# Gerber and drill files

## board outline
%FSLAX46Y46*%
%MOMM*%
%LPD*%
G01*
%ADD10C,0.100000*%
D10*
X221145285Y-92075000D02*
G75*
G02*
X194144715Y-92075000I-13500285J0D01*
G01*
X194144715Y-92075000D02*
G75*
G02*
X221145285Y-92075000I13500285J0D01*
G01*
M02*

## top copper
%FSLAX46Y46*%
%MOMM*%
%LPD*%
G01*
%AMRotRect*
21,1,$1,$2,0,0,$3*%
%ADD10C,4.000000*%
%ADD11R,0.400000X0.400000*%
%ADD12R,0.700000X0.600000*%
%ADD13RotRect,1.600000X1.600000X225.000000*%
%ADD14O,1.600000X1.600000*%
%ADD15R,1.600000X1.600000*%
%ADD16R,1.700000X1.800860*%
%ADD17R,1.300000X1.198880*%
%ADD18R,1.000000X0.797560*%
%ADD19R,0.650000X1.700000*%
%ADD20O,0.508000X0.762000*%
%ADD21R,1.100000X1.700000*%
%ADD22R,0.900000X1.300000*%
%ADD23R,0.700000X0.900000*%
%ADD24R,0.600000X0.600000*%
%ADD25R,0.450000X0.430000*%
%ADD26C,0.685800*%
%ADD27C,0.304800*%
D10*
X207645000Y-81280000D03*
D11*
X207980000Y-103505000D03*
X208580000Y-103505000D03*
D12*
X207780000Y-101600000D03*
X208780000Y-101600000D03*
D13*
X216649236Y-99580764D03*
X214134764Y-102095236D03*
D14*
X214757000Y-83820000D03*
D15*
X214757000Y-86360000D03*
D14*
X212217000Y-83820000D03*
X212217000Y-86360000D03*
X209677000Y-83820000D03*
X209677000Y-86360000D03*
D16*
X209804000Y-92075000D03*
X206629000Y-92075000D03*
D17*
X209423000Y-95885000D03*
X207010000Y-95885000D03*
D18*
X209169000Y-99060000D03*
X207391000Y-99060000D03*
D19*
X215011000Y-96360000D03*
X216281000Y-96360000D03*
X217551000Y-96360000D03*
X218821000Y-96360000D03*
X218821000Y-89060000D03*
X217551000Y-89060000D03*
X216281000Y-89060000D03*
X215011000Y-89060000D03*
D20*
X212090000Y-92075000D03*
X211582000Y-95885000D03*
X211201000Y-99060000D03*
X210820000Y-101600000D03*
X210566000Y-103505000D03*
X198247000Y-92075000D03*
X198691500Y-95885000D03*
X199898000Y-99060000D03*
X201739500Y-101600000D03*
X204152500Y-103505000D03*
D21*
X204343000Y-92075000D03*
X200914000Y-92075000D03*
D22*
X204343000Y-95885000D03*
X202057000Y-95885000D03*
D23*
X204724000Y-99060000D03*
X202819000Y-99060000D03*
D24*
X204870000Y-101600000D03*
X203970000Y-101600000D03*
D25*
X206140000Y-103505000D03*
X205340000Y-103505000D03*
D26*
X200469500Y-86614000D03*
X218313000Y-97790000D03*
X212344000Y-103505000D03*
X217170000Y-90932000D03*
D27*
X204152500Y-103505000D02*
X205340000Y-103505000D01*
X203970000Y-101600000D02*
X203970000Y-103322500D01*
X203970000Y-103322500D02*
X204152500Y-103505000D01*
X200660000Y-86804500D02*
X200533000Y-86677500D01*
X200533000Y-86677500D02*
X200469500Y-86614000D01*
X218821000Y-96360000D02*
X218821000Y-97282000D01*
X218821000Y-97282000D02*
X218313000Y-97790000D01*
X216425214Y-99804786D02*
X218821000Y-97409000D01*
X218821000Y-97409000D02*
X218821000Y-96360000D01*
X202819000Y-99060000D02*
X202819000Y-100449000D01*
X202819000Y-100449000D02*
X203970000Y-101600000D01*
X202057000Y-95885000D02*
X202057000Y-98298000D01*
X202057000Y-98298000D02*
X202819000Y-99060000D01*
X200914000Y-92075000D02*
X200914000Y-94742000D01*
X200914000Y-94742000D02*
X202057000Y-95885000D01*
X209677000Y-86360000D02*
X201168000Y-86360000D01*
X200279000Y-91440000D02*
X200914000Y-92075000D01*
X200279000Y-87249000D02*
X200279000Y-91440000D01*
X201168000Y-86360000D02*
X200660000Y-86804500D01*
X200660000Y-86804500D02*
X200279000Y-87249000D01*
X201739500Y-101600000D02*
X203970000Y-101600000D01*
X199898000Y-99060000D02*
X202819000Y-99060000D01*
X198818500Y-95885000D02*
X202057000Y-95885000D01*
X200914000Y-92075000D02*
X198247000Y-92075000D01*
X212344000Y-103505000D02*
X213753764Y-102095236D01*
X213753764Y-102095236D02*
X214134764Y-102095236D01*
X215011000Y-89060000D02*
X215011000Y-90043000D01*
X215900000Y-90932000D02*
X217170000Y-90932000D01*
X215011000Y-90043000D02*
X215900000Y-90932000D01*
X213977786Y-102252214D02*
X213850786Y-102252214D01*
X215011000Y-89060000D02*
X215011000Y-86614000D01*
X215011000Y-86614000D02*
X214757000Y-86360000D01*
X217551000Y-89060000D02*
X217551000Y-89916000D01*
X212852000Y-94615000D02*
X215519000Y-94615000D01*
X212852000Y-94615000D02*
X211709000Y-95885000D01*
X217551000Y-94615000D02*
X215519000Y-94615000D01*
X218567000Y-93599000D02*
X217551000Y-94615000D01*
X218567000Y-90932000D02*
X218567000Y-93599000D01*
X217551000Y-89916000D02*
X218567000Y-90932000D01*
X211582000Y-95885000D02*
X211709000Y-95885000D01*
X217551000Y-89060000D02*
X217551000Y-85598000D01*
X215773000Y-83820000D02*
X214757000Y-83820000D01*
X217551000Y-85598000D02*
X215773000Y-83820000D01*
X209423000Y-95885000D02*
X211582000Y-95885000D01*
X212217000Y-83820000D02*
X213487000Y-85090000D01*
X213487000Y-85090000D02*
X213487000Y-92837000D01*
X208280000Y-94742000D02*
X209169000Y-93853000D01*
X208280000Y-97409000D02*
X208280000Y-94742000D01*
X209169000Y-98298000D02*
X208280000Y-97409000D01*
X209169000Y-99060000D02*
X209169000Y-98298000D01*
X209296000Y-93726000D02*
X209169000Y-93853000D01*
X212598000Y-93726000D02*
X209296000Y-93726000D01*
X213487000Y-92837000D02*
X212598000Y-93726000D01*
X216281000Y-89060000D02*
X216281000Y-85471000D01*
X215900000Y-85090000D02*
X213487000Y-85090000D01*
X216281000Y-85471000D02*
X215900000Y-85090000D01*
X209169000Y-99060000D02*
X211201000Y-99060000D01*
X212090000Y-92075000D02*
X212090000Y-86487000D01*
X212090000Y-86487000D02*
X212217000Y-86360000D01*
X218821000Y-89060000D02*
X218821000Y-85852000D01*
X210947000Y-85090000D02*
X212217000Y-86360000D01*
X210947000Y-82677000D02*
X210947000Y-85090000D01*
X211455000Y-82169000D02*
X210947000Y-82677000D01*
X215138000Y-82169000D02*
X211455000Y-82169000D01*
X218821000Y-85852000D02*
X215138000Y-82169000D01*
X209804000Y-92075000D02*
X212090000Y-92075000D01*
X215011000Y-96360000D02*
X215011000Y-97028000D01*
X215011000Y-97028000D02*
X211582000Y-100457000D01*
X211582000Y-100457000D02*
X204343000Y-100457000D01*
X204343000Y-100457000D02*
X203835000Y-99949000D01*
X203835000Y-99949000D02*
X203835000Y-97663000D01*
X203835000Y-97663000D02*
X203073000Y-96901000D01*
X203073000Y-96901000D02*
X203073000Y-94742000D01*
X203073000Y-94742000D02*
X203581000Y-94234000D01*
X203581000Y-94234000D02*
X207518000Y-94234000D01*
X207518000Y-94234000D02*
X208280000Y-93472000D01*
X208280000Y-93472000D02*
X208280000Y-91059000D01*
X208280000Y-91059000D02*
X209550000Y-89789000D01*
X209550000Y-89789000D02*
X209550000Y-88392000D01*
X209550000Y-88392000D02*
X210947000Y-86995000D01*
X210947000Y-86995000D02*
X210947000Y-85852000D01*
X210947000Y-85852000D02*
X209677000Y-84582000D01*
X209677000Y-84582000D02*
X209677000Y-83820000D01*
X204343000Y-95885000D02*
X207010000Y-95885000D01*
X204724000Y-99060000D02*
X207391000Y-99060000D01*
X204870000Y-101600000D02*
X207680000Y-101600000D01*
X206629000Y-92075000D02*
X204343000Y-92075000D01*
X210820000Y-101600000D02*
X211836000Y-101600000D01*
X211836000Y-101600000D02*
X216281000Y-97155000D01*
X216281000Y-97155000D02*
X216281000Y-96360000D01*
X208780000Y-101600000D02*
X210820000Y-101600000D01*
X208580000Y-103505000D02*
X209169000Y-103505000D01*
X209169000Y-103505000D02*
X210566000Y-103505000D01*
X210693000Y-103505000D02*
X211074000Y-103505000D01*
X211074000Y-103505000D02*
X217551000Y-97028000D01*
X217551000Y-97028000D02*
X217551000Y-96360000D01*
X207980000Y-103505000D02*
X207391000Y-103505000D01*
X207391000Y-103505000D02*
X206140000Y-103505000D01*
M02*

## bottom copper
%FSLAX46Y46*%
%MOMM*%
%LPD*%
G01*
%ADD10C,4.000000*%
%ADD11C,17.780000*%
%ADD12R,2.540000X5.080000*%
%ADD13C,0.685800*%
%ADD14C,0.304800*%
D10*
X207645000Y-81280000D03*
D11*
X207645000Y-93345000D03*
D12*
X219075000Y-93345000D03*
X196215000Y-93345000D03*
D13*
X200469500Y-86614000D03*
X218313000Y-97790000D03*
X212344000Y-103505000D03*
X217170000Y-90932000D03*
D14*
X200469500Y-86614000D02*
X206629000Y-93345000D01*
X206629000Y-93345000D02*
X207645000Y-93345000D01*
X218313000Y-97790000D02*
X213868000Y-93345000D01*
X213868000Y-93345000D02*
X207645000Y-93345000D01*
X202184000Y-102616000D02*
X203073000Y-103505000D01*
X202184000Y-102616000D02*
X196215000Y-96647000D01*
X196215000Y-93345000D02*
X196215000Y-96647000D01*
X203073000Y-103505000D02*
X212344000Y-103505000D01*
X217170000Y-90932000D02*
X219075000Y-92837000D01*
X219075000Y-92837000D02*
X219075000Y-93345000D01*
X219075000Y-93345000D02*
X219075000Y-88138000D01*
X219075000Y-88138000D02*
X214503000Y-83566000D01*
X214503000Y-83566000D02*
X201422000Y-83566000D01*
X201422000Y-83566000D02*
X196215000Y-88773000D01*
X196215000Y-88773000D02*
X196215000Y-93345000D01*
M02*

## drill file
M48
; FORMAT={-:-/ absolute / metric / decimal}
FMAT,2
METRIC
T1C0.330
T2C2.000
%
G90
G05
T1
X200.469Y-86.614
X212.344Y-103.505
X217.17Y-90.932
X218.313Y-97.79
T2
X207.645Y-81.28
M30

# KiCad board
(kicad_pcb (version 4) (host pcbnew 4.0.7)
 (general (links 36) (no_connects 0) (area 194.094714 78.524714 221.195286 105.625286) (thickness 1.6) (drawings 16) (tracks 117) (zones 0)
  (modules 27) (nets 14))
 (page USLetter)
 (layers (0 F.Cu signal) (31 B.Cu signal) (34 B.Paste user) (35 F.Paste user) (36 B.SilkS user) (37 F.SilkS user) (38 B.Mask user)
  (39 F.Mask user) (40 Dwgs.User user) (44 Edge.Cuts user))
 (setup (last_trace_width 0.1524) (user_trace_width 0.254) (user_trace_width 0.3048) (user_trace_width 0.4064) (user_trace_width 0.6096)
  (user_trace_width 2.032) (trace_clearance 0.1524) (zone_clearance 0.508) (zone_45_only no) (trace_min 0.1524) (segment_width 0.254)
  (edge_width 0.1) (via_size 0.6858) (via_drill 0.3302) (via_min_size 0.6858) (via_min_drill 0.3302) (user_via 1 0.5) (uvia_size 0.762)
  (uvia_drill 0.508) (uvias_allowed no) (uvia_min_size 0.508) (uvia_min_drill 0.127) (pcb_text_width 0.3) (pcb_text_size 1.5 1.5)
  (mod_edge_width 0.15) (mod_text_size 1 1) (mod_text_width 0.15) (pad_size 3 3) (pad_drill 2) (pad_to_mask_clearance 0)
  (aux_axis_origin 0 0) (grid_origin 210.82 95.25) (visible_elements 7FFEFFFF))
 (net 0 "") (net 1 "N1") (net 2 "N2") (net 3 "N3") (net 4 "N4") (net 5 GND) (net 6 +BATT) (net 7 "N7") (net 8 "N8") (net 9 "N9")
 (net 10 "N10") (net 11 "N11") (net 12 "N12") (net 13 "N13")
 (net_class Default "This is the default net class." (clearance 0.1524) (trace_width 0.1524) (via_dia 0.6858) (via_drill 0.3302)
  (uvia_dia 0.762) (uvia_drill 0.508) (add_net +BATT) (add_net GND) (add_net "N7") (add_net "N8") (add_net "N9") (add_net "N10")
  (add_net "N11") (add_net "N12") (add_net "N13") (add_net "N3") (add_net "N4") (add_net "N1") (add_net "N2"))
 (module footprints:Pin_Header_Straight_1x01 (layer F.Cu) (at 207.645 81.28)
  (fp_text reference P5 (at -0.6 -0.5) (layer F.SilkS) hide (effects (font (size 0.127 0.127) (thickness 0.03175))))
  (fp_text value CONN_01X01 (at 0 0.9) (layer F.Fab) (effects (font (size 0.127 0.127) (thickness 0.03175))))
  (pad 1 thru_hole circle (at 0 0) (size 4 4) (drill 2) (layers *.Cu *.Mask)))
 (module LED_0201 (layer F.Cu) (at 208.28 103.505)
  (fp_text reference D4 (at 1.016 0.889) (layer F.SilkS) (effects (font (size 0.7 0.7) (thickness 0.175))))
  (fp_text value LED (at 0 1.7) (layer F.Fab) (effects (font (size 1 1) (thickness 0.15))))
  (pad 1 smd rect (at -0.3 0) (size 0.4 0.4) (layers F.Cu F.Paste F.Mask) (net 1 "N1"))
  (pad 2 smd rect (at 0.3 0) (size 0.4 0.4) (layers F.Cu F.Paste F.Mask) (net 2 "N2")))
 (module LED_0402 (layer F.Cu) (at 208.28 101.6)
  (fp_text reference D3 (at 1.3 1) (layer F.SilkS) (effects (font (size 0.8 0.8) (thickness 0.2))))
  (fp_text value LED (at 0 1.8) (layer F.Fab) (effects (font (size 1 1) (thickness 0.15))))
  (pad 1 smd rect (at -0.5 0) (size 0.7 0.6) (layers F.Cu F.Paste F.Mask) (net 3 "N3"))
  (pad 2 smd rect (at 0.5 0) (size 0.7 0.6) (layers F.Cu F.Paste F.Mask) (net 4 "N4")))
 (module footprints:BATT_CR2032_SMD (layer B.Cu) (at 207.645 93.345 180)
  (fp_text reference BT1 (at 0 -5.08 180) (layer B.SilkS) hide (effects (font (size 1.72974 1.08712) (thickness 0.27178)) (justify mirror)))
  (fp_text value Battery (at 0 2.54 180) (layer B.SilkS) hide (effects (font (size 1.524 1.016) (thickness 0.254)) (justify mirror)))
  (pad 2 smd circle (at 0 0 180) (size 17.78 17.78) (layers B.Cu B.Paste B.Mask) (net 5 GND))
  (pad 1 smd rect (at -11.43 0 180) (size 2.54 5.08) (layers B.Cu B.Paste B.Mask) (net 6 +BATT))
  (pad 1 smd rect (at 11.43 0 180) (size 2.54 5.08) (layers B.Cu B.Paste B.Mask) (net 6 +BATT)))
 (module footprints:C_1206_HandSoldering (layer F.Cu) (at 215.392 100.838 225)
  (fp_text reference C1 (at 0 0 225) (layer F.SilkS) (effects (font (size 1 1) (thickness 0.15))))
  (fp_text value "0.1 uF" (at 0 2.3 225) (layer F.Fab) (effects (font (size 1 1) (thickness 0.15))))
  (pad 1 smd rect (at -1.778 0 225) (size 1.6 1.6) (layers F.Cu F.Paste F.Mask) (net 5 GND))
  (pad 2 smd rect (at 1.778 0 225) (size 1.6 1.6) (layers F.Cu F.Paste F.Mask) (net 6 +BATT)))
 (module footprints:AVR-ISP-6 (layer F.Cu) (at 214.757 83.82 270)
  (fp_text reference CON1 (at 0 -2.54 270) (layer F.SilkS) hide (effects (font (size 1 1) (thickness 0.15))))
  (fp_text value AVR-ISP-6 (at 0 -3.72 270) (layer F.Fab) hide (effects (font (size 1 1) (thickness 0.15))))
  (pad 1 smd oval (at 0 0 270) (size 1.6 1.6) (layers F.Cu F.Paste F.Mask) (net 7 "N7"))
  (pad 2 smd rect (at 2.54 0 270) (size 1.6 1.6) (layers F.Cu F.Paste F.Mask) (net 6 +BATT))
  (pad 3 smd oval (at 0 2.54 270) (size 1.6 1.6) (layers F.Cu F.Paste F.Mask) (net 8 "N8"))
  (pad 4 smd oval (at 2.54 2.54 270) (size 1.6 1.6) (layers F.Cu F.Paste F.Mask) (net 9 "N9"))
  (pad 5 smd oval (at 0 5.08 270) (size 1.6 1.6) (layers F.Cu F.Paste F.Mask) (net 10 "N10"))
  (pad 6 smd oval (at 2.54 5.08 270) (size 1.6 1.6) (layers F.Cu F.Paste F.Mask) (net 5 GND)))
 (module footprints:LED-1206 (layer F.Cu) (at 208.28 92.075)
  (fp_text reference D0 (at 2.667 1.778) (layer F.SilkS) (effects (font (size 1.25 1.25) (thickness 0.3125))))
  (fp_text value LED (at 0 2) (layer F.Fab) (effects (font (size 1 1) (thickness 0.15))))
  (pad 2 smd rect (at 1.524 0 180) (size 1.7 1.80086) (layers F.Cu F.Paste F.Mask) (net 9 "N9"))
  (pad 1 smd rect (at -1.651 0 180) (size 1.7 1.80086) (layers F.Cu F.Paste F.Mask) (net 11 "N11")))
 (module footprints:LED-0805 (layer F.Cu) (at 208.28 95.885)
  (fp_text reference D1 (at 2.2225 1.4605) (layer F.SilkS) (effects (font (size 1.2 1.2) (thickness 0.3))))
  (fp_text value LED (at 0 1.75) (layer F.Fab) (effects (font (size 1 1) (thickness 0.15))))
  (pad 2 smd rect (at 1.143 0 180) (size 1.3 1.19888) (layers F.Cu F.Paste F.Mask) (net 7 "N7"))
  (pad 1 smd rect (at -1.27 0 180) (size 1.3 1.19888) (layers F.Cu F.Paste F.Mask) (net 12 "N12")))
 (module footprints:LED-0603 (layer F.Cu) (at 208.28 99.06)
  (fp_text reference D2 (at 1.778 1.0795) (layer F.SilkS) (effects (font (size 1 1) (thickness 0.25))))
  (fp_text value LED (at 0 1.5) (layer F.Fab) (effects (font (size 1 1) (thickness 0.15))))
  (pad 2 smd rect (at 0.889 0 180) (size 1 0.79756) (layers F.Cu F.Paste F.Mask) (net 8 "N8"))
  (pad 1 smd rect (at -0.889 0 180) (size 1 0.79756) (layers F.Cu F.Paste F.Mask) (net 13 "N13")))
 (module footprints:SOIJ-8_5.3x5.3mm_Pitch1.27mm (layer F.Cu) (at 216.916 92.71 90)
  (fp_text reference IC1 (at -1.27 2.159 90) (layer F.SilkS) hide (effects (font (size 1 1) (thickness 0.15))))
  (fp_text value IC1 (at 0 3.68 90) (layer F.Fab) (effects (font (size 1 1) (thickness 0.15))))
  (pad 1 smd rect (at -3.65 -1.905 90) (size 1.7 0.65) (layers F.Cu F.Paste F.Mask) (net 10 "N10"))
  (pad 2 smd rect (at -3.65 -0.635 90) (size 1.7 0.65) (layers F.Cu F.Paste F.Mask) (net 4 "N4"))
  (pad 3 smd rect (at -3.65 0.635 90) (size 1.7 0.65) (layers F.Cu F.Paste F.Mask) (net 2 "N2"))
  (pad 4 smd rect (at -3.65 1.905 90) (size 1.7 0.65) (layers F.Cu F.Paste F.Mask) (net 5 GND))
  (pad 5 smd rect (at 3.65 1.905 90) (size 1.7 0.65) (layers F.Cu F.Paste F.Mask) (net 9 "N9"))
  (pad 6 smd rect (at 3.65 0.635 90) (size 1.7 0.65) (layers F.Cu F.Paste F.Mask) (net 7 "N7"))
  (pad 7 smd rect (at 3.65 -0.635 90) (size 1.7 0.65) (layers F.Cu F.Paste F.Mask) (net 8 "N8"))
  (pad 8 smd rect (at 3.65 -1.905 90) (size 1.7 0.65) (layers F.Cu F.Paste F.Mask) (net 6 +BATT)))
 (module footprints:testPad (layer F.Cu) (at 212.09 92.075)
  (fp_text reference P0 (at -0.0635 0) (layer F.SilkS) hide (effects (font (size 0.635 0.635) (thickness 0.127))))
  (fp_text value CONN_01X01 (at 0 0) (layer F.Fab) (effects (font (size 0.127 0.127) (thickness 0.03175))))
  (pad 1 smd oval (at 0 0) (size 0.508 0.762) (layers F.Cu F.Paste F.Mask) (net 9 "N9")))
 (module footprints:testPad (layer F.Cu) (at 211.582 95.885)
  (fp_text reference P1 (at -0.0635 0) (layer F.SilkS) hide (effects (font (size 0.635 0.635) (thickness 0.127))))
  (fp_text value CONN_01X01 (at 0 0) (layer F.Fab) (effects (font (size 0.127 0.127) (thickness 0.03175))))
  (pad 1 smd oval (at 0 0) (size 0.508 0.762) (layers F.Cu F.Paste F.Mask) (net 7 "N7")))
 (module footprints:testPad (layer F.Cu) (at 211.201 99.06)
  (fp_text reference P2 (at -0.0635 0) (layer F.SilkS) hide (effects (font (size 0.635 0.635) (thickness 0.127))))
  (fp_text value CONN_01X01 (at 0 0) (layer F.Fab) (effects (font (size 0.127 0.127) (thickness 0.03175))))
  (pad 1 smd oval (at 0 0) (size 0.508 0.762) (layers F.Cu F.Paste F.Mask) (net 8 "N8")))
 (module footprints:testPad (layer F.Cu) (at 210.82 101.6)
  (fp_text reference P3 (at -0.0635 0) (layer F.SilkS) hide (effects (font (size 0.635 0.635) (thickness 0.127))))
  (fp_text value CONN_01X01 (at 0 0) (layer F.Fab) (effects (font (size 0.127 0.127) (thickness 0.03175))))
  (pad 1 smd oval (at 0 0) (size 0.508 0.762) (layers F.Cu F.Paste F.Mask) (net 4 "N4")))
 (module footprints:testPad (layer F.Cu) (at 210.566 103.505)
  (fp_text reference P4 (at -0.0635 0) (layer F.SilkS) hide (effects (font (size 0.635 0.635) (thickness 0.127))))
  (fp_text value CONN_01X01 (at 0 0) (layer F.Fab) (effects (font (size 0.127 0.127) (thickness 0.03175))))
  (pad 1 smd oval (at 0 0) (size 0.508 0.762) (layers F.Cu F.Paste F.Mask) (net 2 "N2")))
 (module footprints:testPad (layer F.Cu) (at 198.247 92.075)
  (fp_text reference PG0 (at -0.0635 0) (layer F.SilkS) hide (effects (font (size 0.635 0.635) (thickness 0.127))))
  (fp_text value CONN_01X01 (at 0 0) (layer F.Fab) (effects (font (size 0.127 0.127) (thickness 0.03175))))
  (pad 1 smd oval (at 0 0) (size 0.508 0.762) (layers F.Cu F.Paste F.Mask) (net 5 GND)))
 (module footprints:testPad (layer F.Cu) (at 198.6915 95.885)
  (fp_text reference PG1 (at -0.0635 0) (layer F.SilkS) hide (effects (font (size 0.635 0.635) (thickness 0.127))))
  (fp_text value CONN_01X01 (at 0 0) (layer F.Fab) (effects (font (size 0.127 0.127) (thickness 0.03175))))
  (pad 1 smd oval (at 0 0) (size 0.508 0.762) (layers F.Cu F.Paste F.Mask) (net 5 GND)))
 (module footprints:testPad (layer F.Cu) (at 199.898 99.06)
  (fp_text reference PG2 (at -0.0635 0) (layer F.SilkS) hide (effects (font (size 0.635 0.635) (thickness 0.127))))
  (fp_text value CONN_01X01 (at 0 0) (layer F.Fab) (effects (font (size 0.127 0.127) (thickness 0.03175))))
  (pad 1 smd oval (at 0 0) (size 0.508 0.762) (layers F.Cu F.Paste F.Mask) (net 5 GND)))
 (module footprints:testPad (layer F.Cu) (at 201.7395 101.6)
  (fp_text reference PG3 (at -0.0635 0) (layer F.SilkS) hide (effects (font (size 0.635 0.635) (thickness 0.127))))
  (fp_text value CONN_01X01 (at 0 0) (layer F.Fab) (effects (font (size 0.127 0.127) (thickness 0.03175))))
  (pad 1 smd oval (at 0 0) (size 0.508 0.762) (layers F.Cu F.Paste F.Mask) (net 5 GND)))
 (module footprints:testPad (layer F.Cu) (at 204.1525 103.505)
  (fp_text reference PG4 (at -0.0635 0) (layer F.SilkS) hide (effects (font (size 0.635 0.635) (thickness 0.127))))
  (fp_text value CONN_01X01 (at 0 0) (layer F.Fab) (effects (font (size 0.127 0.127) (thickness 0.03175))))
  (pad 1 smd oval (at 0 0) (size 0.508 0.762) (layers F.Cu F.Paste F.Mask) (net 5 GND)))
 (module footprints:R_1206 (layer F.Cu) (at 202.565 92.075 180)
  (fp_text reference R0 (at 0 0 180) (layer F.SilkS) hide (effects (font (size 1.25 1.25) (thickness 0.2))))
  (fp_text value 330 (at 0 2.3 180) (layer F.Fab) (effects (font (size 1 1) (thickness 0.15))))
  (pad 1 smd rect (at -1.778 0 180) (size 1.1 1.7) (layers F.Cu F.Paste F.Mask) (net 11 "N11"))
  (pad 2 smd rect (at 1.651 0 180) (size 1.1 1.7) (layers F.Cu F.Paste F.Mask) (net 5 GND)))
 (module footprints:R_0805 (layer F.Cu) (at 203.2 95.885 180)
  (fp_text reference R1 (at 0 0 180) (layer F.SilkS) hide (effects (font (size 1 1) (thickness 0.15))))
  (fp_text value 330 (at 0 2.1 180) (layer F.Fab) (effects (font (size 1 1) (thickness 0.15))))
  (pad 1 smd rect (at -1.143 0 180) (size 0.9 1.3) (layers F.Cu F.Paste F.Mask) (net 12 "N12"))
  (pad 2 smd rect (at 1.143 0 180) (size 0.9 1.3) (layers F.Cu F.Paste F.Mask) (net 5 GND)))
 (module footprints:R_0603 (layer F.Cu) (at 203.835 99.06 180)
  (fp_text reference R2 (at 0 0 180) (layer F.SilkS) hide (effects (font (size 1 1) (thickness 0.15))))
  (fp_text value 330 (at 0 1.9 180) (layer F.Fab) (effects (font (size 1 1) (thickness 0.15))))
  (pad 1 smd rect (at -0.889 0 180) (size 0.7 0.9) (layers F.Cu F.Paste F.Mask) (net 13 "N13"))
  (pad 2 smd rect (at 1.016 0 180) (size 0.7 0.9) (layers F.Cu F.Paste F.Mask) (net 5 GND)))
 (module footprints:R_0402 (layer F.Cu) (at 204.47 101.6 180)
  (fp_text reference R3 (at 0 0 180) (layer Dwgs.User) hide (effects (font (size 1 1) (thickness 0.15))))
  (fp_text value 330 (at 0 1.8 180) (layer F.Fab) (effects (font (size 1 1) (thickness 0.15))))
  (pad 1 smd rect (at -0.4 0 180) (size 0.6 0.6) (layers F.Cu F.Paste F.Mask) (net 3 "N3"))
  (pad 2 smd rect (at 0.5 0 180) (size 0.6 0.6) (layers F.Cu F.Paste F.Mask) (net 5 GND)))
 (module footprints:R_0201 (layer F.Cu) (at 205.74 103.505 180)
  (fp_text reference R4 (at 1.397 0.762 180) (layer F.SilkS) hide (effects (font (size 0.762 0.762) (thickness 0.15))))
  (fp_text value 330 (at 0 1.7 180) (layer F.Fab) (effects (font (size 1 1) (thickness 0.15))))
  (pad 1 smd rect (at -0.4 0 180) (size 0.45 0.43) (layers F.Cu F.Paste F.Mask) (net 1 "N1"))
  (pad 2 smd rect (at 0.4 0 180) (size 0.45 0.43) (layers F.Cu F.Paste F.Mask) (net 5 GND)))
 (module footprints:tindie (layer F.Cu) (at 208.534 88.9)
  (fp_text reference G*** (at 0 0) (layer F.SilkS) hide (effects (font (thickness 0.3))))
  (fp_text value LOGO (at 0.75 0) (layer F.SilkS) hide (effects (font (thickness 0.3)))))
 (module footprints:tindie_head (layer F.Cu) (at 200.914 86.36)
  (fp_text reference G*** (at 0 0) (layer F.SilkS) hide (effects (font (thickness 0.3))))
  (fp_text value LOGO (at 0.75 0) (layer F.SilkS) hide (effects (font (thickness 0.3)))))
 (gr_circle (center 207.645 92.075) (end 197.485 83.185) (layer Edge.Cuts) (width 0.1))
 (segment (start 204.1525 103.505) (end 205.34 103.505) (width 0.3048) (layer F.Cu) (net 5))
 (segment (start 203.97 101.6) (end 203.97 103.3225) (width 0.3048) (layer F.Cu) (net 5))
 (segment (start 203.97 103.3225) (end 204.1525 103.505) (width 0.3048) (layer F.Cu) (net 5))
 (segment (start 200.66 86.8045) (end 200.533 86.6775) (width 0.3048) (layer F.Cu) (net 5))
 (segment (start 200.4695 86.614) (end 206.629 93.345) (width 0.3048) (layer B.Cu) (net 5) (status 20))
 (via (at 200.4695 86.614) (size 0.6858) (drill 0.3302) (layers F.Cu B.Cu) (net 5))
 (segment (start 200.533 86.6775) (end 200.4695 86.614) (width 0.3048) (layer F.Cu) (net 5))
 (segment (start 206.629 93.345) (end 207.645 93.345) (width 0.3048) (layer B.Cu) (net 5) (status 30))
 (segment (start 218.821 96.36) (end 218.821 97.282) (width 0.3048) (layer F.Cu) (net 5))
 (segment (start 218.313 97.79) (end 213.868 93.345) (width 0.3048) (layer B.Cu) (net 5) (status 20))
 (via (at 218.313 97.79) (size 0.6858) (drill 0.3302) (layers F.Cu B.Cu) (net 5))
 (segment (start 218.821 97.282) (end 218.313 97.79) (width 0.3048) (layer F.Cu) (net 5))
 (segment (start 213.868 93.345) (end 207.645 93.345) (width 0.3048) (layer B.Cu) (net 5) (status 30))
 (segment (start 216.425214 99.804786) (end 218.821 97.409) (width 0.3048) (layer F.Cu) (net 5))
 (segment (start 218.821 97.409) (end 218.821 96.36) (width 0.3048) (layer F.Cu) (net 5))
 (segment (start 202.819 99.06) (end 202.819 100.449) (width 0.3048) (layer F.Cu) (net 5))
 (segment (start 202.819 100.449) (end 203.97 101.6) (width 0.3048) (layer F.Cu) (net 5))
 (segment (start 202.057 95.885) (end 202.057 98.298) (width 0.3048) (layer F.Cu) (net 5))
 (segment (start 202.057 98.298) (end 202.819 99.06) (width 0.3048) (layer F.Cu) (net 5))
 (segment (start 200.914 92.075) (end 200.914 94.742) (width 0.3048) (layer F.Cu) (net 5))
 (segment (start 200.914 94.742) (end 202.057 95.885) (width 0.3048) (layer F.Cu) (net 5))
 (segment (start 209.677 86.36) (end 201.168 86.36) (width 0.3048) (layer F.Cu) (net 5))
 (segment (start 200.279 91.44) (end 200.914 92.075) (width 0.3048) (layer F.Cu) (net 5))
 (segment (start 200.279 87.249) (end 200.279 91.44) (width 0.3048) (layer F.Cu) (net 5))
 (segment (start 201.168 86.36) (end 200.66 86.8045) (width 0.3048) (layer F.Cu) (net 5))
 (segment (start 200.66 86.8045) (end 200.279 87.249) (width 0.3048) (layer F.Cu) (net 5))
 (segment (start 201.7395 101.6) (end 203.97 101.6) (width 0.3048) (layer F.Cu) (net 5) (status 10))
 (segment (start 199.898 99.06) (end 202.819 99.06) (width 0.3048) (layer F.Cu) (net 5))
 (segment (start 198.8185 95.885) (end 202.057 95.885) (width 0.3048) (layer F.Cu) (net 5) (status 10))
 (segment (start 200.914 92.075) (end 198.247 92.075) (width 0.3048) (layer F.Cu) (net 5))
 (segment (start 202.184 102.616) (end 203.073 103.505) (width 0.3048) (layer B.Cu) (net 6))
 (segment (start 202.184 102.616) (end 196.215 96.647) (width 0.3048) (layer B.Cu) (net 6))
 (segment (start 196.215 93.345) (end 196.215 96.647) (width 0.3048) (layer B.Cu) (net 6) (status 10))
 (segment (start 212.344 103.505) (end 213.753764 102.095236) (width 0.3048) (layer F.Cu) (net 6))
 (via (at 212.344 103.505) (size 0.6858) (drill 0.3302) (layers F.Cu B.Cu) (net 6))
 (segment (start 203.073 103.505) (end 212.344 103.505) (width 0.3048) (layer B.Cu) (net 6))
 (segment (start 213.753764 102.095236) (end 214.134764 102.095236) (width 0.3048) (layer F.Cu) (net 6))
 (segment (start 215.011 89.06) (end 215.011 90.043) (width 0.3048) (layer F.Cu) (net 6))
 (segment (start 217.17 90.932) (end 219.075 92.837) (width 0.3048) (layer B.Cu) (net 6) (status 20))
 (via (at 217.17 90.932) (size 0.6858) (drill 0.3302) (layers F.Cu B.Cu) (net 6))
 (segment (start 215.9 90.932) (end 217.17 90.932) (width 0.3048) (layer F.Cu) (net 6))
 (segment (start 215.011 90.043) (end 215.9 90.932) (width 0.3048) (layer F.Cu) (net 6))
 (segment (start 219.075 92.837) (end 219.075 93.345) (width 0.3048) (layer B.Cu) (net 6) (status 30))
 (segment (start 219.075 93.345) (end 219.075 88.138) (width 0.3048) (layer B.Cu) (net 6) (status 10))
 (segment (start 219.075 88.138) (end 214.503 83.566) (width 0.3048) (layer B.Cu) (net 6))
 (segment (start 214.503 83.566) (end 201.422 83.566) (width 0.3048) (layer B.Cu) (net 6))
 (segment (start 201.422 83.566) (end 196.215 88.773) (width 0.3048) (layer B.Cu) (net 6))
 (segment (start 196.215 88.773) (end 196.215 93.345) (width 0.3048) (layer B.Cu) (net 6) (status 20))
 (segment (start 213.977786 102.252214) (end 213.850786 102.252214) (width 0.3048) (layer F.Cu) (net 6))
 (segment (start 215.011 89.06) (end 215.011 86.614) (width 0.3048) (layer F.Cu) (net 6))
 (segment (start 215.011 86.614) (end 214.757 86.36) (width 0.3048) (layer F.Cu) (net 6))
 (segment (start 217.551 89.06) (end 217.551 89.916) (width 0.3048) (layer F.Cu) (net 7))
 (segment (start 212.852 94.615) (end 215.519 94.615) (width 0.3048) (layer F.Cu) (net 7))
 (segment (start 212.852 94.615) (end 211.709 95.885) (width 0.3048) (layer F.Cu) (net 7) (status 20))
 (segment (start 217.551 94.615) (end 215.519 94.615) (width 0.3048) (layer F.Cu) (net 7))
 (segment (start 218.567 93.599) (end 217.551 94.615) (width 0.3048) (layer F.Cu) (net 7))
 (segment (start 218.567 90.932) (end 218.567 93.599) (width 0.3048) (layer F.Cu) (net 7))
 (segment (start 217.551 89.916) (end 218.567 90.932) (width 0.3048) (layer F.Cu) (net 7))
 (segment (start 211.582 95.885) (end 211.709 95.885) (width 0.3048) (layer F.Cu) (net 7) (status 30))
 (segment (start 217.551 89.06) (end 217.551 85.598) (width 0.3048) (layer F.Cu) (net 7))
 (segment (start 215.773 83.82) (end 214.757 83.82) (width 0.3048) (layer F.Cu) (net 7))
 (segment (start 217.551 85.598) (end 215.773 83.82) (width 0.3048) (layer F.Cu) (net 7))
 (segment (start 209.423 95.885) (end 211.582 95.885) (width 0.3048) (layer F.Cu) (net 7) (status 20))
 (segment (start 212.217 83.82) (end 213.487 85.09) (width 0.3048) (layer F.Cu) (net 8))
 (segment (start 213.487 85.09) (end 213.487 92.837) (width 0.3048) (layer F.Cu) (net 8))
 (segment (start 208.28 94.742) (end 209.169 93.853) (width 0.3048) (layer F.Cu) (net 8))
 (segment (start 208.28 97.409) (end 208.28 94.742) (width 0.3048) (layer F.Cu) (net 8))
 (segment (start 209.169 98.298) (end 208.28 97.409) (width 0.3048) (layer F.Cu) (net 8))
 (segment (start 209.169 99.06) (end 209.169 98.298) (width 0.3048) (layer F.Cu) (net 8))
 (segment (start 209.296 93.726) (end 209.169 93.853) (width 0.3048) (layer F.Cu) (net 8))
 (segment (start 212.598 93.726) (end 209.296 93.726) (width 0.3048) (layer F.Cu) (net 8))
 (segment (start 213.487 92.837) (end 212.598 93.726) (width 0.3048) (layer F.Cu) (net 8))
 (segment (start 216.281 89.06) (end 216.281 85.471) (width 0.3048) (layer F.Cu) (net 8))
 (segment (start 215.9 85.09) (end 213.487 85.09) (width 0.3048) (layer F.Cu) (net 8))
 (segment (start 216.281 85.471) (end 215.9 85.09) (width 0.3048) (layer F.Cu) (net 8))
 (segment (start 209.169 99.06) (end 211.201 99.06) (width 0.3048) (layer F.Cu) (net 8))
 (segment (start 212.09 92.075) (end 212.09 86.487) (width 0.3048) (layer F.Cu) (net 9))
 (segment (start 212.09 86.487) (end 212.217 86.36) (width 0.3048) (layer F.Cu) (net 9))
 (segment (start 218.821 89.06) (end 218.821 85.852) (width 0.3048) (layer F.Cu) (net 9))
 (segment (start 210.947 85.09) (end 212.217 86.36) (width 0.3048) (layer F.Cu) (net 9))
 (segment (start 210.947 82.677) (end 210.947 85.09) (width 0.3048) (layer F.Cu) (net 9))
 (segment (start 211.455 82.169) (end 210.947 82.677) (width 0.3048) (layer F.Cu) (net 9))
 (segment (start 215.138 82.169) (end 211.455 82.169) (width 0.3048) (layer F.Cu) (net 9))
 (segment (start 218.821 85.852) (end 215.138 82.169) (width 0.3048) (layer F.Cu) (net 9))
 (segment (start 209.804 92.075) (end 212.09 92.075) (width 0.3048) (layer F.Cu) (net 9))
 (segment (start 215.011 96.36) (end 215.011 97.028) (width 0.3048) (layer F.Cu) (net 10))
 (segment (start 215.011 97.028) (end 211.582 100.457) (width 0.3048) (layer F.Cu) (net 10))
 (segment (start 211.582 100.457) (end 204.343 100.457) (width 0.3048) (layer F.Cu) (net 10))
 (segment (start 204.343 100.457) (end 203.835 99.949) (width 0.3048) (layer F.Cu) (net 10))
 (segment (start 203.835 99.949) (end 203.835 97.663) (width 0.3048) (layer F.Cu) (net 10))
 (segment (start 203.835 97.663) (end 203.073 96.901) (width 0.3048) (layer F.Cu) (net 10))
 (segment (start 203.073 96.901) (end 203.073 94.742) (width 0.3048) (layer F.Cu) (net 10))
 (segment (start 203.073 94.742) (end 203.581 94.234) (width 0.3048) (layer F.Cu) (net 10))
 (segment (start 203.581 94.234) (end 207.518 94.234) (width 0.3048) (layer F.Cu) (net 10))
 (segment (start 207.518 94.234) (end 208.28 93.472) (width 0.3048) (layer F.Cu) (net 10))
 (segment (start 208.28 93.472) (end 208.28 91.059) (width 0.3048) (layer F.Cu) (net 10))
 (segment (start 208.28 91.059) (end 209.55 89.789) (width 0.3048) (layer F.Cu) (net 10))
 (segment (start 209.55 89.789) (end 209.55 88.392) (width 0.3048) (layer F.Cu) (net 10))
 (segment (start 209.55 88.392) (end 210.947 86.995) (width 0.3048) (layer F.Cu) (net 10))
 (segment (start 210.947 86.995) (end 210.947 85.852) (width 0.3048) (layer F.Cu) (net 10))
 (segment (start 210.947 85.852) (end 209.677 84.582) (width 0.3048) (layer F.Cu) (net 10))
 (segment (start 209.677 84.582) (end 209.677 83.82) (width 0.3048) (layer F.Cu) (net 10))
 (segment (start 204.343 95.885) (end 207.01 95.885) (width 0.3048) (layer F.Cu) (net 12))
 (segment (start 204.724 99.06) (end 207.391 99.06) (width 0.3048) (layer F.Cu) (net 13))
 (segment (start 204.87 101.6) (end 207.68 101.6) (width 0.3048) (layer F.Cu) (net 3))
 (segment (start 206.629 92.075) (end 204.343 92.075) (width 0.3048) (layer F.Cu) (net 11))
 (segment (start 210.82 101.6) (end 211.836 101.6) (width 0.3048) (layer F.Cu) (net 4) (status 10))
 (segment (start 211.836 101.6) (end 216.281 97.155) (width 0.3048) (layer F.Cu) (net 4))
 (segment (start 216.281 97.155) (end 216.281 96.36) (width 0.3048) (layer F.Cu) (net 4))
 (segment (start 208.78 101.6) (end 210.82 101.6) (width 0.3048) (layer F.Cu) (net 4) (status 20))
 (segment (start 208.58 103.505) (end 209.169 103.505) (width 0.3048) (layer F.Cu) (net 2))
 (segment (start 209.169 103.505) (end 210.566 103.505) (width 0.3048) (layer F.Cu) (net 2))
 (segment (start 210.693 103.505) (end 211.074 103.505) (width 0.3048) (layer F.Cu) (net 2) (status 10))
 (segment (start 211.074 103.505) (end 217.551 97.028) (width 0.3048) (layer F.Cu) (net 2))
 (segment (start 217.551 97.028) (end 217.551 96.36) (width 0.3048) (layer F.Cu) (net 2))
 (segment (start 207.98 103.505) (end 207.391 103.505) (width 0.3048) (layer F.Cu) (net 1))
 (segment (start 207.391 103.505) (end 206.14 103.505) (width 0.3048) (layer F.Cu) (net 1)))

